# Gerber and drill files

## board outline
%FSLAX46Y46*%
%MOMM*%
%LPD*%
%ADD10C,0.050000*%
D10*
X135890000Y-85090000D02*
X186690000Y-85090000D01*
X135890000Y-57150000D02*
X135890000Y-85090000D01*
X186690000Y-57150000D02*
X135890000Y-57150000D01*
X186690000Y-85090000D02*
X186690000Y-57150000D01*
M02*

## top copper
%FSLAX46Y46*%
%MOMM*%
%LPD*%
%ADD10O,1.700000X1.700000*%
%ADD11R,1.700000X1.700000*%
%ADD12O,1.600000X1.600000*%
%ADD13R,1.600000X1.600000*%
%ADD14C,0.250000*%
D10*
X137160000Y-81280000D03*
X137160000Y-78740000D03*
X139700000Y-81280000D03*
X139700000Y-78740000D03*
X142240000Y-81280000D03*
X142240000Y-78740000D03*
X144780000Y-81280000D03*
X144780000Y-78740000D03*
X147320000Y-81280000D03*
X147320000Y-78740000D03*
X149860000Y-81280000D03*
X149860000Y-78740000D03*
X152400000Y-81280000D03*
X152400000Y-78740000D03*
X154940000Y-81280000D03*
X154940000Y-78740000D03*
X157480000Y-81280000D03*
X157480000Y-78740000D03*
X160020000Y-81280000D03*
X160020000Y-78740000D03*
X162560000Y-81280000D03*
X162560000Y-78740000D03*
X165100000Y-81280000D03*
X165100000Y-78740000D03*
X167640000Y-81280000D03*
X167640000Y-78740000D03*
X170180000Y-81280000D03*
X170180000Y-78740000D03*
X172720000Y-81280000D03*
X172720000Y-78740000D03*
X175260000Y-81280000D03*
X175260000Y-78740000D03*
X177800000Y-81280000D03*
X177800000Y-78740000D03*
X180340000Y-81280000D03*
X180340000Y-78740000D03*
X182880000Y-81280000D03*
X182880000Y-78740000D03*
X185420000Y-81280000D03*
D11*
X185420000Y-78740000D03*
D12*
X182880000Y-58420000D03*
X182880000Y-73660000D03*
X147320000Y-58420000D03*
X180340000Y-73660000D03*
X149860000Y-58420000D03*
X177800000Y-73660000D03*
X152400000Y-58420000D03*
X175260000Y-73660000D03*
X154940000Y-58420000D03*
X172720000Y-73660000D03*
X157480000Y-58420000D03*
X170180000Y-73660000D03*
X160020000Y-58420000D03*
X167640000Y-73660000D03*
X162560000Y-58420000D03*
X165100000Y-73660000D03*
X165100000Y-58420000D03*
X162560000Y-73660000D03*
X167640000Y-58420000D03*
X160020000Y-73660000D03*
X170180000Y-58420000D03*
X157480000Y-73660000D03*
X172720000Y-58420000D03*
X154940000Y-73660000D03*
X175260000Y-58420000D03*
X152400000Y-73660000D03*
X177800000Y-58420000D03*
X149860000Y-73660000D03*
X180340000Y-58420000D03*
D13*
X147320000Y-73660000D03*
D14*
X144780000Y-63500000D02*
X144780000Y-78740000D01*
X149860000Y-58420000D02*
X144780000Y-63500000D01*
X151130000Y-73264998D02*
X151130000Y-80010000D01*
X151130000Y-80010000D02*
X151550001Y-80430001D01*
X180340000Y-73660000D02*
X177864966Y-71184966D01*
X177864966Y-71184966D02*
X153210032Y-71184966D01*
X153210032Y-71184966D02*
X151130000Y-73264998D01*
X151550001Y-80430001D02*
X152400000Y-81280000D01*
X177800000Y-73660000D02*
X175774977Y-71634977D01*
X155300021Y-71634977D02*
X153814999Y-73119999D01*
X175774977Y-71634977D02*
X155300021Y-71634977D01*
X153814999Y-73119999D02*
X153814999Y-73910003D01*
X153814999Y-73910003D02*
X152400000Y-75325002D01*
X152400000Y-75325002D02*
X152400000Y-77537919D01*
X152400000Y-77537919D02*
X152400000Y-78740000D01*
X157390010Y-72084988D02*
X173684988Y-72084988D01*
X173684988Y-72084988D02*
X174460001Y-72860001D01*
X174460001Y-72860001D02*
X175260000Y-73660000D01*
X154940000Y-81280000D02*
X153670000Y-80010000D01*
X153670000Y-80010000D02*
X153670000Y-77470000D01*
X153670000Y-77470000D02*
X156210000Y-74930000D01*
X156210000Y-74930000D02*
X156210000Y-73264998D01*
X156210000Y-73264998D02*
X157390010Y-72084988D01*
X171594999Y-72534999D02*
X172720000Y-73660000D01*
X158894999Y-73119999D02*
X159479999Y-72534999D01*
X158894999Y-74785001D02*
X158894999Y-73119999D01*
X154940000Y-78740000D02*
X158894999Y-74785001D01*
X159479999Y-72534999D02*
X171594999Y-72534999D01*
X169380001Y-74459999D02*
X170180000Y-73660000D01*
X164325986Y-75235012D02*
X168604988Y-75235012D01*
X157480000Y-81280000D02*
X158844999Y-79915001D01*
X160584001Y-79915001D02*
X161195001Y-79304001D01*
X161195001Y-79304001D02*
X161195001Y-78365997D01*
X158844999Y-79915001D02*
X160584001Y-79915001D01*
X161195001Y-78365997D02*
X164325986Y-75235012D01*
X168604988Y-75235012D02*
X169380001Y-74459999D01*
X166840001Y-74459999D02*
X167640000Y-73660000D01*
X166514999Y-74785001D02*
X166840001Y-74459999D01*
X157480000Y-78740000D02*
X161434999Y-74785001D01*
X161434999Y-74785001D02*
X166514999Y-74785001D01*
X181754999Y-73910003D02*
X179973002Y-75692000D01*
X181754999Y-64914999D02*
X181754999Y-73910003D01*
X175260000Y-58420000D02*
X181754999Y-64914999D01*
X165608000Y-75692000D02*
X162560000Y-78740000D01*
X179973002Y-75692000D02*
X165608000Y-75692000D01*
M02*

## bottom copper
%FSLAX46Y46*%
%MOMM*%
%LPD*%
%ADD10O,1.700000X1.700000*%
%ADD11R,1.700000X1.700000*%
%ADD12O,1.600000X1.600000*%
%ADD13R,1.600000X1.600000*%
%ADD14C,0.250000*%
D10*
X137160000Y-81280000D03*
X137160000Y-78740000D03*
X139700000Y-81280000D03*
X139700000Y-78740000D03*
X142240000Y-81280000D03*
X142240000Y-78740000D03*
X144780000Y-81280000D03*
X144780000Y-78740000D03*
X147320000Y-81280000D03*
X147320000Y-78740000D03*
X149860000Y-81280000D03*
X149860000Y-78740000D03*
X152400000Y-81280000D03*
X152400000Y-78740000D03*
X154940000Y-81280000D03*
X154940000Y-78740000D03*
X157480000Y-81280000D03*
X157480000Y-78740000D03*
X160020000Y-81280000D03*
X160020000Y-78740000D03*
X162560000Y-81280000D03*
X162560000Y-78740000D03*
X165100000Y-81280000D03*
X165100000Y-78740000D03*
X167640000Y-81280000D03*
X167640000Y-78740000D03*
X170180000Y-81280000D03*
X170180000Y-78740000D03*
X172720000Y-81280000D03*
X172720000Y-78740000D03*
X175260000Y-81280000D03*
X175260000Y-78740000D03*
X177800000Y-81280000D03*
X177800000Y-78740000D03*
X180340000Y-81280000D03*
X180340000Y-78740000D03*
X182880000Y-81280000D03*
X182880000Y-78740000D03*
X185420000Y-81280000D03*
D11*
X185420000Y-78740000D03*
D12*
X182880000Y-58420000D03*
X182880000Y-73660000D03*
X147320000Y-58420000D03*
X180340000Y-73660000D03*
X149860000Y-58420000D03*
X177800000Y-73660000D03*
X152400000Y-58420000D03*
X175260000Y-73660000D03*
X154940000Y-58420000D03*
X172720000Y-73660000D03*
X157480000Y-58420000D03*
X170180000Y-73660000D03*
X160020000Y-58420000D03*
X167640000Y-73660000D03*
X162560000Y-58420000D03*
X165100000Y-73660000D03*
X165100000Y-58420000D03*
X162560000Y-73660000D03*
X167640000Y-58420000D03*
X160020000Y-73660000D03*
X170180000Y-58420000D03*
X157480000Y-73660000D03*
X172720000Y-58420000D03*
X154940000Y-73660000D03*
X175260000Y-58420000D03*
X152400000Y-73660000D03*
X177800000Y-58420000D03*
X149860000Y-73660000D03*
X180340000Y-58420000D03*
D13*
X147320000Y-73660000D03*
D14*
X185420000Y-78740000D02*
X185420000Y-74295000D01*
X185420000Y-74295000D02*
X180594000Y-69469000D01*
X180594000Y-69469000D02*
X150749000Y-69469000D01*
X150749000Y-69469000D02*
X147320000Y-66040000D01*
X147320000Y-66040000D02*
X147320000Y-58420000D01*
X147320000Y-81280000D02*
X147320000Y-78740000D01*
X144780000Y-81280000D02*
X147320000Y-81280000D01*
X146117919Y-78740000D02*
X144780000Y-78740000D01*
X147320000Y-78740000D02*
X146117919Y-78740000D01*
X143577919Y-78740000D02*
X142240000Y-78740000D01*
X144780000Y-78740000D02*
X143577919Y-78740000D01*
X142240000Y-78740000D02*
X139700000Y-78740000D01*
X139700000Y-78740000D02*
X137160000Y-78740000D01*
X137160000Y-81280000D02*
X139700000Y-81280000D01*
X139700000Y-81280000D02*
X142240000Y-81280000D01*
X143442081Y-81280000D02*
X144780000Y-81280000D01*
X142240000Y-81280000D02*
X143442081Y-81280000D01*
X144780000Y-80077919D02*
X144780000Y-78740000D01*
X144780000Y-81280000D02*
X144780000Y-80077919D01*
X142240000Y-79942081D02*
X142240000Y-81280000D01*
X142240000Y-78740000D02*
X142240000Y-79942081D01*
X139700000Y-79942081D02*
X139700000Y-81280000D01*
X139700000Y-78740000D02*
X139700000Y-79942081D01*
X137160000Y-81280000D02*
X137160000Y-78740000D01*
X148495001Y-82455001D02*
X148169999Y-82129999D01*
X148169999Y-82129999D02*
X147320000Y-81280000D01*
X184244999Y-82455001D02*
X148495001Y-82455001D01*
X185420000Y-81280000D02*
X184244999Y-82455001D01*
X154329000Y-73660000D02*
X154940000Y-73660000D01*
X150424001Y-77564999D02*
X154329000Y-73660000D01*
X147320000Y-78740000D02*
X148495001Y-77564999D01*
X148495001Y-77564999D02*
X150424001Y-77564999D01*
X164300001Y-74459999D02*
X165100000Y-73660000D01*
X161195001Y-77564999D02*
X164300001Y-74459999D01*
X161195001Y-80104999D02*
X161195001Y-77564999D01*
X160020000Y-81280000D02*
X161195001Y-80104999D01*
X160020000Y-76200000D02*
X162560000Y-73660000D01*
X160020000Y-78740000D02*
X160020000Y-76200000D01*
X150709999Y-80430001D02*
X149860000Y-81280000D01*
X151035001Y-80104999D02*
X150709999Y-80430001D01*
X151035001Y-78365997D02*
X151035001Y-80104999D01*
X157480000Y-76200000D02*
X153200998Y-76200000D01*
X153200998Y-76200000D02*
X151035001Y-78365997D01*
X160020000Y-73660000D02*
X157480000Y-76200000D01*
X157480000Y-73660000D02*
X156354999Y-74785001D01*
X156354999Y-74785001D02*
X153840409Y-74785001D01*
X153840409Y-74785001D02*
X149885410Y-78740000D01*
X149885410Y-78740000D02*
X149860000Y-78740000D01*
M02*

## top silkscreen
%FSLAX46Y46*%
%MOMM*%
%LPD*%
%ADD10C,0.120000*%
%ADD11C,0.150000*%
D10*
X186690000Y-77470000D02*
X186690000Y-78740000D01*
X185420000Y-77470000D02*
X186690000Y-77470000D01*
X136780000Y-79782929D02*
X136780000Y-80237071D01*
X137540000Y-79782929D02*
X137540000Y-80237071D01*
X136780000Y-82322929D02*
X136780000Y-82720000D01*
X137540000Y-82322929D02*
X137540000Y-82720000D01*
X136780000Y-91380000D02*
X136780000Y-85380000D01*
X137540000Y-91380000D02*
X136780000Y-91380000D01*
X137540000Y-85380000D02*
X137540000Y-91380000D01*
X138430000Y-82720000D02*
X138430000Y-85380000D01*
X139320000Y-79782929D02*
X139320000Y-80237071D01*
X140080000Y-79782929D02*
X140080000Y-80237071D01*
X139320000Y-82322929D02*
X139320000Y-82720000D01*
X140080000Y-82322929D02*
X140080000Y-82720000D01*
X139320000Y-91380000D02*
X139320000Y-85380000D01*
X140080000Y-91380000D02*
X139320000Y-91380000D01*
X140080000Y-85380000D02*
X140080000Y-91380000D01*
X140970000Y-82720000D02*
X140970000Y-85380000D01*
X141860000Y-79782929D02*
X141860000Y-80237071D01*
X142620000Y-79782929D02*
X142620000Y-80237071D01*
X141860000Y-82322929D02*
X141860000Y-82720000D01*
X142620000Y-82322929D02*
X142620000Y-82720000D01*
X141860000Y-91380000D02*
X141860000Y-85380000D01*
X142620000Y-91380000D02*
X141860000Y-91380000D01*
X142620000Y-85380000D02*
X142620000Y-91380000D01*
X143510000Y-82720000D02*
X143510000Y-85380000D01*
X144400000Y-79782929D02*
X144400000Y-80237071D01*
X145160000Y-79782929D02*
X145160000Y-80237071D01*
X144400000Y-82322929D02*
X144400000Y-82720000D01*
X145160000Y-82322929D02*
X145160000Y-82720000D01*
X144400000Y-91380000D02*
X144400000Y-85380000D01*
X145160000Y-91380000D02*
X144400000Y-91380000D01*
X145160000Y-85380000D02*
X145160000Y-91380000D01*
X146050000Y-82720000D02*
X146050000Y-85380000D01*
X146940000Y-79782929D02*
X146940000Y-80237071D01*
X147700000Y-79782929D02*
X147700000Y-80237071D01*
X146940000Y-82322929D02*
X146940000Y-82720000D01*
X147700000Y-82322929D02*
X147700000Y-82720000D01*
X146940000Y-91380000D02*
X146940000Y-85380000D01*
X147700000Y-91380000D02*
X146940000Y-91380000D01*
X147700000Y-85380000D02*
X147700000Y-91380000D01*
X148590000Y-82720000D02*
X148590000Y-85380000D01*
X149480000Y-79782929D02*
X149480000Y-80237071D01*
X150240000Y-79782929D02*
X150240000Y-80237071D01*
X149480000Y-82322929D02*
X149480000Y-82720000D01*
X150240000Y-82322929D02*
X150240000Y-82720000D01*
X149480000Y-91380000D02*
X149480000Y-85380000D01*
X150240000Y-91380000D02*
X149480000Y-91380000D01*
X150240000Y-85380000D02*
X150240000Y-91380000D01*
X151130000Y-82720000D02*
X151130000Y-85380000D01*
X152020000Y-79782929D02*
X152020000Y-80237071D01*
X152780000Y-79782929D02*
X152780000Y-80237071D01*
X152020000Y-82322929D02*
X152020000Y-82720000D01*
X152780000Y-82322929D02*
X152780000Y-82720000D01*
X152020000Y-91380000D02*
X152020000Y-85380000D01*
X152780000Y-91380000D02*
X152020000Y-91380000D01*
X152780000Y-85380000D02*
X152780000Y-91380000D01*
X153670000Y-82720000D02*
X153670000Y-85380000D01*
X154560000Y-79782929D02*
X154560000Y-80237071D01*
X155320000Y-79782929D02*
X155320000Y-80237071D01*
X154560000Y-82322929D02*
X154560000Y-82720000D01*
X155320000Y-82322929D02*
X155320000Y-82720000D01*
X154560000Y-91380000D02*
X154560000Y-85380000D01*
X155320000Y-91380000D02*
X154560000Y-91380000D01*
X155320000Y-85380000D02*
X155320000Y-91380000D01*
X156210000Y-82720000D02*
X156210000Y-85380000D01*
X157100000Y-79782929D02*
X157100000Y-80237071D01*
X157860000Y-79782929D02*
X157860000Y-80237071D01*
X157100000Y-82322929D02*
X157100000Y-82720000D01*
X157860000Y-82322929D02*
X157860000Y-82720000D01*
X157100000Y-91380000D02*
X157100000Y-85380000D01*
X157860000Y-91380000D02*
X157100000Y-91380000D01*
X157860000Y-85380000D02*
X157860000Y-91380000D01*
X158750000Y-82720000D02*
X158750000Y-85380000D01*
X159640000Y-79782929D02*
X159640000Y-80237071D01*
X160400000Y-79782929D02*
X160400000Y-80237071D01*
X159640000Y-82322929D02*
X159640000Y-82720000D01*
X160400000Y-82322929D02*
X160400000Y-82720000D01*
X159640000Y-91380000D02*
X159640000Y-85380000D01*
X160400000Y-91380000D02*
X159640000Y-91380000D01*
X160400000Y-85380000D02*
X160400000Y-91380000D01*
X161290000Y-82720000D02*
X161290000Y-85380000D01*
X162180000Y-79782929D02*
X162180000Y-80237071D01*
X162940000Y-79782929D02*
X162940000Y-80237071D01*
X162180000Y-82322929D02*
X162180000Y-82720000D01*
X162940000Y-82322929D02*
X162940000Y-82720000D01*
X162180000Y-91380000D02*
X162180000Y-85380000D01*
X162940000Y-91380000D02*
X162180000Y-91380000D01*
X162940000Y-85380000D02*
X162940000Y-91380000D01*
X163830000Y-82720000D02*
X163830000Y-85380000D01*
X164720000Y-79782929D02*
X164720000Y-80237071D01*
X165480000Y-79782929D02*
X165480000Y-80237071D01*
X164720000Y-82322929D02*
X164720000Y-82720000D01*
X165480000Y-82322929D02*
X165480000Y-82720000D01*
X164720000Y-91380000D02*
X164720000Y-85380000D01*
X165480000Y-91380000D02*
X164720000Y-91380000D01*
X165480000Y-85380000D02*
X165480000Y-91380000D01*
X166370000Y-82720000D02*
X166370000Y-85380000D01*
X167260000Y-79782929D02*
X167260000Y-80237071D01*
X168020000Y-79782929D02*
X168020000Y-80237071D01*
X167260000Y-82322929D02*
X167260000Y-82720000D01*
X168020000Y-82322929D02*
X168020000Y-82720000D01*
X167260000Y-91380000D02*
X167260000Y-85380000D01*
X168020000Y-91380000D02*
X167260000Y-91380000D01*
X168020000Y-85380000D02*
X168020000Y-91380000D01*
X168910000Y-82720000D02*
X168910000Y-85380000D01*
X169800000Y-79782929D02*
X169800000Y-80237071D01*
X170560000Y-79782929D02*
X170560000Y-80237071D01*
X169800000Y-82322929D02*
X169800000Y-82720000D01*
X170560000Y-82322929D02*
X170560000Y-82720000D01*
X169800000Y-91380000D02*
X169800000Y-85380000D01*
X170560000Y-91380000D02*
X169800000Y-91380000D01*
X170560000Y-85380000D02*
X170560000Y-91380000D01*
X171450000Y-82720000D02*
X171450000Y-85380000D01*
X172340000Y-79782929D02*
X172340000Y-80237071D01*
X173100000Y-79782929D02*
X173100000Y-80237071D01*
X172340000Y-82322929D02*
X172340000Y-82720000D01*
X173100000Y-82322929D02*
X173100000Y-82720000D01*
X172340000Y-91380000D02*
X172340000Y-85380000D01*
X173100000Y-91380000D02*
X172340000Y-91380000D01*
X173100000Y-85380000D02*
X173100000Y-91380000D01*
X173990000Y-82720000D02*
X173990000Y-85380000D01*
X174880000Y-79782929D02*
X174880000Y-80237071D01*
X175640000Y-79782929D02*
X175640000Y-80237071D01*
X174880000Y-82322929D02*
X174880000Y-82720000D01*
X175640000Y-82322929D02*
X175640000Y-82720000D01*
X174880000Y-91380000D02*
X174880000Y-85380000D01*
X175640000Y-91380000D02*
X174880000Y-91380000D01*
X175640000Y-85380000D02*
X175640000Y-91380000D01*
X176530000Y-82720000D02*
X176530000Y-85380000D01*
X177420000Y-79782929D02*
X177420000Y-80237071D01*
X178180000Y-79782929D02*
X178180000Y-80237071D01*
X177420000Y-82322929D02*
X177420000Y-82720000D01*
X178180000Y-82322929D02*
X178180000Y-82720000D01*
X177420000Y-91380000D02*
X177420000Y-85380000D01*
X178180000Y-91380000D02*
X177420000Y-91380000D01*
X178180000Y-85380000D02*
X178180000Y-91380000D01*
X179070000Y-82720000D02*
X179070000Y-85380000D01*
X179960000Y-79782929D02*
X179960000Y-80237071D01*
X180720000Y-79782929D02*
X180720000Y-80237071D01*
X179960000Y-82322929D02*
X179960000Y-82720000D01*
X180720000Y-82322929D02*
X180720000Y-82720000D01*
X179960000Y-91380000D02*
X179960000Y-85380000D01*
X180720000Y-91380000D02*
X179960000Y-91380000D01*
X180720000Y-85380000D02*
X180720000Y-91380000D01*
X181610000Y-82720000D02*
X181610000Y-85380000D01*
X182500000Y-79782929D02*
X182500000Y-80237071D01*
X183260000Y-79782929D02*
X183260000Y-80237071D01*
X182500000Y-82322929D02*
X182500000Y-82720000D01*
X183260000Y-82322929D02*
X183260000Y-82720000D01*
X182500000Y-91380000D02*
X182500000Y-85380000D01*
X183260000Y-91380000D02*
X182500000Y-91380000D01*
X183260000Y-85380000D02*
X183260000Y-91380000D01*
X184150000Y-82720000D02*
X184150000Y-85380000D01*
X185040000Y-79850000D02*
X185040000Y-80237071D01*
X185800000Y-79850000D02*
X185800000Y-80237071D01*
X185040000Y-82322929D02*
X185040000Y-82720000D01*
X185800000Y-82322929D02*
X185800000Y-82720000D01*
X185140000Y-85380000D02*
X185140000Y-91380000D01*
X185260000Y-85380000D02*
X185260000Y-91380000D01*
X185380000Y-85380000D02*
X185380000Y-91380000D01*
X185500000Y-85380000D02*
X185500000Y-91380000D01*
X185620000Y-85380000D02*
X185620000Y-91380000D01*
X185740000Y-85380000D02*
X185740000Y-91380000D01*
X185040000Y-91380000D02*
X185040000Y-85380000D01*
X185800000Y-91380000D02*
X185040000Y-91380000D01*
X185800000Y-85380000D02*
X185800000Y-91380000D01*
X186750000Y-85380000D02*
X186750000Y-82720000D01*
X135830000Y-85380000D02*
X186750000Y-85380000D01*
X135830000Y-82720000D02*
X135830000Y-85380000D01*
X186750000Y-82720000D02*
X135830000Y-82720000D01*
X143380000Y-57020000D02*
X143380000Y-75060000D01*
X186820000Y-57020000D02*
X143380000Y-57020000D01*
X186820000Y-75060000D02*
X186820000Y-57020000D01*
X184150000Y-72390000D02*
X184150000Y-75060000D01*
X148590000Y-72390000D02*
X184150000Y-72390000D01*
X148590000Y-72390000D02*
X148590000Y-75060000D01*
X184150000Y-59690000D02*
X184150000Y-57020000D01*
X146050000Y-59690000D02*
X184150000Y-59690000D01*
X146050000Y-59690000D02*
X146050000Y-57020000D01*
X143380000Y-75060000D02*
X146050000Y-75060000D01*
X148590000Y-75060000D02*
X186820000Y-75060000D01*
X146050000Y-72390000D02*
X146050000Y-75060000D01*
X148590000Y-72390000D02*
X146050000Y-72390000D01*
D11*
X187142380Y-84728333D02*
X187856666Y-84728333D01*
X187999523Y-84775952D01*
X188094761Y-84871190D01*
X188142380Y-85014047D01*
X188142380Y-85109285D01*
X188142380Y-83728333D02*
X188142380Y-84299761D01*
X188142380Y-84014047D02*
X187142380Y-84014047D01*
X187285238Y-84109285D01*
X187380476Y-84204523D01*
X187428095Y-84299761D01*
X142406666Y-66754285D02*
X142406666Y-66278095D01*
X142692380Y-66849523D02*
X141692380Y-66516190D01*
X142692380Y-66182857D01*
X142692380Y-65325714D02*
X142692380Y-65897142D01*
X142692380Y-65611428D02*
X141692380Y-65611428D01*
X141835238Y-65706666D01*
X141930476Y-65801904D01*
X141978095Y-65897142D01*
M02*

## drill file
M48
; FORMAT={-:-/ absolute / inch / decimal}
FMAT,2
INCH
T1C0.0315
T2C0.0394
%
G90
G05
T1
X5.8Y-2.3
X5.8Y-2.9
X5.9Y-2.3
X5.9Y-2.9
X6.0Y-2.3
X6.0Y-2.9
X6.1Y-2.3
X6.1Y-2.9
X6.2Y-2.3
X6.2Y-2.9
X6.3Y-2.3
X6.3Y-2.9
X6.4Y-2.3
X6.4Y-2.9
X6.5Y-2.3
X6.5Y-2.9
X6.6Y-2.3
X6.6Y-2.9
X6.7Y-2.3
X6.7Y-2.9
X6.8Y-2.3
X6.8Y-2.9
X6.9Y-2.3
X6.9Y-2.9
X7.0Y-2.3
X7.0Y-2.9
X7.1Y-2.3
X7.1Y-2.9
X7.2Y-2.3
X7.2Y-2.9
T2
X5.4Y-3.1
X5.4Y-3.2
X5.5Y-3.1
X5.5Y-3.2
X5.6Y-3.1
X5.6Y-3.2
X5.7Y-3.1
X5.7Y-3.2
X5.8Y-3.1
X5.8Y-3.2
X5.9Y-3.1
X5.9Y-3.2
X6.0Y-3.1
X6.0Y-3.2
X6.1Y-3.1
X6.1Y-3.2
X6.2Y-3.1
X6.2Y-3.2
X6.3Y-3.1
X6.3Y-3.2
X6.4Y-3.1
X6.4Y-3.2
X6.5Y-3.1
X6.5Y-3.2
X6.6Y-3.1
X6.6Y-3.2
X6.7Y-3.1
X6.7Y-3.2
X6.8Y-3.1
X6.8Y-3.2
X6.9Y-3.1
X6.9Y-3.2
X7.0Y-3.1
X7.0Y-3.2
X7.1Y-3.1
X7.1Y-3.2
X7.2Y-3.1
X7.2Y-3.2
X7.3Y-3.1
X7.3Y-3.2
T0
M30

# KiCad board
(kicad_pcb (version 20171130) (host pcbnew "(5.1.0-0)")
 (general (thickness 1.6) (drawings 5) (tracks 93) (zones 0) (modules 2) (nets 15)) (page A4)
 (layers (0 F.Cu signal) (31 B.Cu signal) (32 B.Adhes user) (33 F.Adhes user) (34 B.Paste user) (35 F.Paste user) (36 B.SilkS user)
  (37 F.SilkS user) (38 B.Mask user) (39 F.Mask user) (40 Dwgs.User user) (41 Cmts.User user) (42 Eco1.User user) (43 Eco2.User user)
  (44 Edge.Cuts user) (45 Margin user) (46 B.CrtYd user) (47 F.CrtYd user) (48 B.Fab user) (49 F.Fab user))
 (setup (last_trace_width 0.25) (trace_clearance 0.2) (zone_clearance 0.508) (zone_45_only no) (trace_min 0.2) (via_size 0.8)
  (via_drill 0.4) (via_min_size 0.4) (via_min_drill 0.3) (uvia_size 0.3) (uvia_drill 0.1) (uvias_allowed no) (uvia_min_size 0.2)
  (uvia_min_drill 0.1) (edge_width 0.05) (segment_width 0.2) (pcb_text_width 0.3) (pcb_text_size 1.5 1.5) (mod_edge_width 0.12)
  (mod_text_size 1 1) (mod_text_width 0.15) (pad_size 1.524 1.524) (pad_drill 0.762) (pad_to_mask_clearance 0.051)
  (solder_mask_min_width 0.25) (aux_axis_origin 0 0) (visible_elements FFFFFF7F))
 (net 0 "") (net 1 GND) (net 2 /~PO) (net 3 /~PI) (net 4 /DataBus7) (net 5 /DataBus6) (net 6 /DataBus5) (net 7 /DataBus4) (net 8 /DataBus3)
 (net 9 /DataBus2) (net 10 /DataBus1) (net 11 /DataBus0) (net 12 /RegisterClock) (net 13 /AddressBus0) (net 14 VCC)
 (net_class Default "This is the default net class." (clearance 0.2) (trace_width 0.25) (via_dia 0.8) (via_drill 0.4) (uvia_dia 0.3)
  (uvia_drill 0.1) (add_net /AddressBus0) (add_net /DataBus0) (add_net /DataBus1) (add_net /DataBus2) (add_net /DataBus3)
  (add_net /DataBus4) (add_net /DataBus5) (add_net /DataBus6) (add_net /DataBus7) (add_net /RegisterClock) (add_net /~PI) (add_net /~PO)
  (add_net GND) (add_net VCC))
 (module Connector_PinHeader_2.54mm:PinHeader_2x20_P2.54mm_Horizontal (layer F.Cu) (at 185.42 78.74 270)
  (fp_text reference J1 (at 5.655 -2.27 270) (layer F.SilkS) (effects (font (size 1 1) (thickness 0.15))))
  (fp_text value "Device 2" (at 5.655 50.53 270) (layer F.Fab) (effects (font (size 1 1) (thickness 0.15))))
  (fp_line (start -1.27 -1.27) (end 0 -1.27) (layer F.SilkS) (width 0.12))
  (fp_line (start -1.27 0) (end -1.27 -1.27) (layer F.SilkS) (width 0.12))
  (fp_line (start 1.042929 48.64) (end 1.497071 48.64) (layer F.SilkS) (width 0.12))
  (fp_line (start 1.042929 47.88) (end 1.497071 47.88) (layer F.SilkS) (width 0.12))
  (fp_line (start 3.582929 48.64) (end 3.98 48.64) (layer F.SilkS) (width 0.12))
  (fp_line (start 3.582929 47.88) (end 3.98 47.88) (layer F.SilkS) (width 0.12))
  (fp_line (start 12.64 48.64) (end 6.64 48.64) (layer F.SilkS) (width 0.12))
  (fp_line (start 12.64 47.88) (end 12.64 48.64) (layer F.SilkS) (width 0.12))
  (fp_line (start 6.64 47.88) (end 12.64 47.88) (layer F.SilkS) (width 0.12))
  (fp_line (start 3.98 46.99) (end 6.64 46.99) (layer F.SilkS) (width 0.12))
  (fp_line (start 1.042929 46.1) (end 1.497071 46.1) (layer F.SilkS) (width 0.12))
  (fp_line (start 1.042929 45.34) (end 1.497071 45.34) (layer F.SilkS) (width 0.12))
  (fp_line (start 3.582929 46.1) (end 3.98 46.1) (layer F.SilkS) (width 0.12))
  (fp_line (start 3.582929 45.34) (end 3.98 45.34) (layer F.SilkS) (width 0.12))
  (fp_line (start 12.64 46.1) (end 6.64 46.1) (layer F.SilkS) (width 0.12))
  (fp_line (start 12.64 45.34) (end 12.64 46.1) (layer F.SilkS) (width 0.12))
  (fp_line (start 6.64 45.34) (end 12.64 45.34) (layer F.SilkS) (width 0.12))
  (fp_line (start 3.98 44.45) (end 6.64 44.45) (layer F.SilkS) (width 0.12))
  (fp_line (start 1.042929 43.56) (end 1.497071 43.56) (layer F.SilkS) (width 0.12))
  (fp_line (start 1.042929 42.8) (end 1.497071 42.8) (layer F.SilkS) (width 0.12))
  (fp_line (start 3.582929 43.56) (end 3.98 43.56) (layer F.SilkS) (width 0.12))
  (fp_line (start 3.582929 42.8) (end 3.98 42.8) (layer F.SilkS) (width 0.12))
  (fp_line (start 12.64 43.56) (end 6.64 43.56) (layer F.SilkS) (width 0.12))
  (fp_line (start 12.64 42.8) (end 12.64 43.56) (layer F.SilkS) (width 0.12))
  (fp_line (start 6.64 42.8) (end 12.64 42.8) (layer F.SilkS) (width 0.12))
  (fp_line (start 3.98 41.91) (end 6.64 41.91) (layer F.SilkS) (width 0.12))
  (fp_line (start 1.042929 41.02) (end 1.497071 41.02) (layer F.SilkS) (width 0.12))
  (fp_line (start 1.042929 40.26) (end 1.497071 40.26) (layer F.SilkS) (width 0.12))
  (fp_line (start 3.582929 41.02) (end 3.98 41.02) (layer F.SilkS) (width 0.12))
  (fp_line (start 3.582929 40.26) (end 3.98 40.26) (layer F.SilkS) (width 0.12))
  (fp_line (start 12.64 41.02) (end 6.64 41.02) (layer F.SilkS) (width 0.12))
  (fp_line (start 12.64 40.26) (end 12.64 41.02) (layer F.SilkS) (width 0.12))
  (fp_line (start 6.64 40.26) (end 12.64 40.26) (layer F.SilkS) (width 0.12))
  (fp_line (start 3.98 39.37) (end 6.64 39.37) (layer F.SilkS) (width 0.12))
  (fp_line (start 1.042929 38.48) (end 1.497071 38.48) (layer F.SilkS) (width 0.12))
  (fp_line (start 1.042929 37.72) (end 1.497071 37.72) (layer F.SilkS) (width 0.12))
  (fp_line (start 3.582929 38.48) (end 3.98 38.48) (layer F.SilkS) (width 0.12))
  (fp_line (start 3.582929 37.72) (end 3.98 37.72) (layer F.SilkS) (width 0.12))
  (fp_line (start 12.64 38.48) (end 6.64 38.48) (layer F.SilkS) (width 0.12))
  (fp_line (start 12.64 37.72) (end 12.64 38.48) (layer F.SilkS) (width 0.12))
  (fp_line (start 6.64 37.72) (end 12.64 37.72) (layer F.SilkS) (width 0.12))
  (fp_line (start 3.98 36.83) (end 6.64 36.83) (layer F.SilkS) (width 0.12))
  (fp_line (start 1.042929 35.94) (end 1.497071 35.94) (layer F.SilkS) (width 0.12))
  (fp_line (start 1.042929 35.18) (end 1.497071 35.18) (layer F.SilkS) (width 0.12))
  (fp_line (start 3.582929 35.94) (end 3.98 35.94) (layer F.SilkS) (width 0.12))
  (fp_line (start 3.582929 35.18) (end 3.98 35.18) (layer F.SilkS) (width 0.12))
  (fp_line (start 12.64 35.94) (end 6.64 35.94) (layer F.SilkS) (width 0.12))
  (fp_line (start 12.64 35.18) (end 12.64 35.94) (layer F.SilkS) (width 0.12))
  (fp_line (start 6.64 35.18) (end 12.64 35.18) (layer F.SilkS) (width 0.12))
  (fp_line (start 3.98 34.29) (end 6.64 34.29) (layer F.SilkS) (width 0.12))
  (fp_line (start 1.042929 33.4) (end 1.497071 33.4) (layer F.SilkS) (width 0.12))
  (fp_line (start 1.042929 32.64) (end 1.497071 32.64) (layer F.SilkS) (width 0.12))
  (fp_line (start 3.582929 33.4) (end 3.98 33.4) (layer F.SilkS) (width 0.12))
  (fp_line (start 3.582929 32.64) (end 3.98 32.64) (layer F.SilkS) (width 0.12))
  (fp_line (start 12.64 33.4) (end 6.64 33.4) (layer F.SilkS) (width 0.12))
  (fp_line (start 12.64 32.64) (end 12.64 33.4) (layer F.SilkS) (width 0.12))
  (fp_line (start 6.64 32.64) (end 12.64 32.64) (layer F.SilkS) (width 0.12))
  (fp_line (start 3.98 31.75) (end 6.64 31.75) (layer F.SilkS) (width 0.12))
  (fp_line (start 1.042929 30.86) (end 1.497071 30.86) (layer F.SilkS) (width 0.12))
  (fp_line (start 1.042929 30.1) (end 1.497071 30.1) (layer F.SilkS) (width 0.12))
  (fp_line (start 3.582929 30.86) (end 3.98 30.86) (layer F.SilkS) (width 0.12))
  (fp_line (start 3.582929 30.1) (end 3.98 30.1) (layer F.SilkS) (width 0.12))
  (fp_line (start 12.64 30.86) (end 6.64 30.86) (layer F.SilkS) (width 0.12))
  (fp_line (start 12.64 30.1) (end 12.64 30.86) (layer F.SilkS) (width 0.12))
  (fp_line (start 6.64 30.1) (end 12.64 30.1) (layer F.SilkS) (width 0.12))
  (fp_line (start 3.98 29.21) (end 6.64 29.21) (layer F.SilkS) (width 0.12))
  (fp_line (start 1.042929 28.32) (end 1.497071 28.32) (layer F.SilkS) (width 0.12))
  (fp_line (start 1.042929 27.56) (end 1.497071 27.56) (layer F.SilkS) (width 0.12))
  (fp_line (start 3.582929 28.32) (end 3.98 28.32) (layer F.SilkS) (width 0.12))
  (fp_line (start 3.582929 27.56) (end 3.98 27.56) (layer F.SilkS) (width 0.12))
  (fp_line (start 12.64 28.32) (end 6.64 28.32) (layer F.SilkS) (width 0.12))
  (fp_line (start 12.64 27.56) (end 12.64 28.32) (layer F.SilkS) (width 0.12))
  (fp_line (start 6.64 27.56) (end 12.64 27.56) (layer F.SilkS) (width 0.12))
  (fp_line (start 3.98 26.67) (end 6.64 26.67) (layer F.SilkS) (width 0.12))
  (fp_line (start 1.042929 25.78) (end 1.497071 25.78) (layer F.SilkS) (width 0.12))
  (fp_line (start 1.042929 25.02) (end 1.497071 25.02) (layer F.SilkS) (width 0.12))
  (fp_line (start 3.582929 25.78) (end 3.98 25.78) (layer F.SilkS) (width 0.12))
  (fp_line (start 3.582929 25.02) (end 3.98 25.02) (layer F.SilkS) (width 0.12))
  (fp_line (start 12.64 25.78) (end 6.64 25.78) (layer F.SilkS) (width 0.12))
  (fp_line (start 12.64 25.02) (end 12.64 25.78) (layer F.SilkS) (width 0.12))
  (fp_line (start 6.64 25.02) (end 12.64 25.02) (layer F.SilkS) (width 0.12))
  (fp_line (start 3.98 24.13) (end 6.64 24.13) (layer F.SilkS) (width 0.12))
  (fp_line (start 1.042929 23.24) (end 1.497071 23.24) (layer F.SilkS) (width 0.12))
  (fp_line (start 1.042929 22.48) (end 1.497071 22.48) (layer F.SilkS) (width 0.12))
  (fp_line (start 3.582929 23.24) (end 3.98 23.24) (layer F.SilkS) (width 0.12))
  (fp_line (start 3.582929 22.48) (end 3.98 22.48) (layer F.SilkS) (width 0.12))
  (fp_line (start 12.64 23.24) (end 6.64 23.24) (layer F.SilkS) (width 0.12))
  (fp_line (start 12.64 22.48) (end 12.64 23.24) (layer F.SilkS) (width 0.12))
  (fp_line (start 6.64 22.48) (end 12.64 22.48) (layer F.SilkS) (width 0.12))
  (fp_line (start 3.98 21.59) (end 6.64 21.59) (layer F.SilkS) (width 0.12))
  (fp_line (start 1.042929 20.7) (end 1.497071 20.7) (layer F.SilkS) (width 0.12))
  (fp_line (start 1.042929 19.94) (end 1.497071 19.94) (layer F.SilkS) (width 0.12))
  (fp_line (start 3.582929 20.7) (end 3.98 20.7) (layer F.SilkS) (width 0.12))
  (fp_line (start 3.582929 19.94) (end 3.98 19.94) (layer F.SilkS) (width 0.12))
  (fp_line (start 12.64 20.7) (end 6.64 20.7) (layer F.SilkS) (width 0.12))
  (fp_line (start 12.64 19.94) (end 12.64 20.7) (layer F.SilkS) (width 0.12))
  (fp_line (start 6.64 19.94) (end 12.64 19.94) (layer F.SilkS) (width 0.12))
  (fp_line (start 3.98 19.05) (end 6.64 19.05) (layer F.SilkS) (width 0.12))
  (fp_line (start 1.042929 18.16) (end 1.497071 18.16) (layer F.SilkS) (width 0.12))
  (fp_line (start 1.042929 17.4) (end 1.497071 17.4) (layer F.SilkS) (width 0.12))
  (fp_line (start 3.582929 18.16) (end 3.98 18.16) (layer F.SilkS) (width 0.12))
  (fp_line (start 3.582929 17.4) (end 3.98 17.4) (layer F.SilkS) (width 0.12))
  (fp_line (start 12.64 18.16) (end 6.64 18.16) (layer F.SilkS) (width 0.12))
  (fp_line (start 12.64 17.4) (end 12.64 18.16) (layer F.SilkS) (width 0.12))
  (fp_line (start 6.64 17.4) (end 12.64 17.4) (layer F.SilkS) (width 0.12))
  (fp_line (start 3.98 16.51) (end 6.64 16.51) (layer F.SilkS) (width 0.12))
  (fp_line (start 1.042929 15.62) (end 1.497071 15.62) (layer F.SilkS) (width 0.12))
  (fp_line (start 1.042929 14.86) (end 1.497071 14.86) (layer F.SilkS) (width 0.12))
  (fp_line (start 3.582929 15.62) (end 3.98 15.62) (layer F.SilkS) (width 0.12))
  (fp_line (start 3.582929 14.86) (end 3.98 14.86) (layer F.SilkS) (width 0.12))
  (fp_line (start 12.64 15.62) (end 6.64 15.62) (layer F.SilkS) (width 0.12))
  (fp_line (start 12.64 14.86) (end 12.64 15.62) (layer F.SilkS) (width 0.12))
  (fp_line (start 6.64 14.86) (end 12.64 14.86) (layer F.SilkS) (width 0.12))
  (fp_line (start 3.98 13.97) (end 6.64 13.97) (layer F.SilkS) (width 0.12))
  (fp_line (start 1.042929 13.08) (end 1.497071 13.08) (layer F.SilkS) (width 0.12))
  (fp_line (start 1.042929 12.32) (end 1.497071 12.32) (layer F.SilkS) (width 0.12))
  (fp_line (start 3.582929 13.08) (end 3.98 13.08) (layer F.SilkS) (width 0.12))
  (fp_line (start 3.582929 12.32) (end 3.98 12.32) (layer F.SilkS) (width 0.12))
  (fp_line (start 12.64 13.08) (end 6.64 13.08) (layer F.SilkS) (width 0.12))
  (fp_line (start 12.64 12.32) (end 12.64 13.08) (layer F.SilkS) (width 0.12))
  (fp_line (start 6.64 12.32) (end 12.64 12.32) (layer F.SilkS) (width 0.12))
  (fp_line (start 3.98 11.43) (end 6.64 11.43) (layer F.SilkS) (width 0.12))
  (fp_line (start 1.042929 10.54) (end 1.497071 10.54) (layer F.SilkS) (width 0.12))
  (fp_line (start 1.042929 9.78) (end 1.497071 9.78) (layer F.SilkS) (width 0.12))
  (fp_line (start 3.582929 10.54) (end 3.98 10.54) (layer F.SilkS) (width 0.12))
  (fp_line (start 3.582929 9.78) (end 3.98 9.78) (layer F.SilkS) (width 0.12))
  (fp_line (start 12.64 10.54) (end 6.64 10.54) (layer F.SilkS) (width 0.12))
  (fp_line (start 12.64 9.78) (end 12.64 10.54) (layer F.SilkS) (width 0.12))
  (fp_line (start 6.64 9.78) (end 12.64 9.78) (layer F.SilkS) (width 0.12))
  (fp_line (start 3.98 8.89) (end 6.64 8.89) (layer F.SilkS) (width 0.12))
  (fp_line (start 1.042929 8) (end 1.497071 8) (layer F.SilkS) (width 0.12))
  (fp_line (start 1.042929 7.24) (end 1.497071 7.24) (layer F.SilkS) (width 0.12))
  (fp_line (start 3.582929 8) (end 3.98 8) (layer F.SilkS) (width 0.12))
  (fp_line (start 3.582929 7.24) (end 3.98 7.24) (layer F.SilkS) (width 0.12))
  (fp_line (start 12.64 8) (end 6.64 8) (layer F.SilkS) (width 0.12))
  (fp_line (start 12.64 7.24) (end 12.64 8) (layer F.SilkS) (width 0.12))
  (fp_line (start 6.64 7.24) (end 12.64 7.24) (layer F.SilkS) (width 0.12))
  (fp_line (start 3.98 6.35) (end 6.64 6.35) (layer F.SilkS) (width 0.12))
  (fp_line (start 1.042929 5.46) (end 1.497071 5.46) (layer F.SilkS) (width 0.12))
  (fp_line (start 1.042929 4.7) (end 1.497071 4.7) (layer F.SilkS) (width 0.12))
  (fp_line (start 3.582929 5.46) (end 3.98 5.46) (layer F.SilkS) (width 0.12))
  (fp_line (start 3.582929 4.7) (end 3.98 4.7) (layer F.SilkS) (width 0.12))
  (fp_line (start 12.64 5.46) (end 6.64 5.46) (layer F.SilkS) (width 0.12))
  (fp_line (start 12.64 4.7) (end 12.64 5.46) (layer F.SilkS) (width 0.12))
  (fp_line (start 6.64 4.7) (end 12.64 4.7) (layer F.SilkS) (width 0.12))
  (fp_line (start 3.98 3.81) (end 6.64 3.81) (layer F.SilkS) (width 0.12))
  (fp_line (start 1.042929 2.92) (end 1.497071 2.92) (layer F.SilkS) (width 0.12))
  (fp_line (start 1.042929 2.16) (end 1.497071 2.16) (layer F.SilkS) (width 0.12))
  (fp_line (start 3.582929 2.92) (end 3.98 2.92) (layer F.SilkS) (width 0.12))
  (fp_line (start 3.582929 2.16) (end 3.98 2.16) (layer F.SilkS) (width 0.12))
  (fp_line (start 12.64 2.92) (end 6.64 2.92) (layer F.SilkS) (width 0.12))
  (fp_line (start 12.64 2.16) (end 12.64 2.92) (layer F.SilkS) (width 0.12))
  (fp_line (start 6.64 2.16) (end 12.64 2.16) (layer F.SilkS) (width 0.12))
  (fp_line (start 3.98 1.27) (end 6.64 1.27) (layer F.SilkS) (width 0.12))
  (fp_line (start 1.11 0.38) (end 1.497071 0.38) (layer F.SilkS) (width 0.12))
  (fp_line (start 1.11 -0.38) (end 1.497071 -0.38) (layer F.SilkS) (width 0.12))
  (fp_line (start 3.582929 0.38) (end 3.98 0.38) (layer F.SilkS) (width 0.12))
  (fp_line (start 3.582929 -0.38) (end 3.98 -0.38) (layer F.SilkS) (width 0.12))
  (fp_line (start 6.64 0.28) (end 12.64 0.28) (layer F.SilkS) (width 0.12))
  (fp_line (start 6.64 0.16) (end 12.64 0.16) (layer F.SilkS) (width 0.12))
  (fp_line (start 6.64 0.04) (end 12.64 0.04) (layer F.SilkS) (width 0.12))
  (fp_line (start 6.64 -0.08) (end 12.64 -0.08) (layer F.SilkS) (width 0.12))
  (fp_line (start 6.64 -0.2) (end 12.64 -0.2) (layer F.SilkS) (width 0.12))
  (fp_line (start 6.64 -0.32) (end 12.64 -0.32) (layer F.SilkS) (width 0.12))
  (fp_line (start 12.64 0.38) (end 6.64 0.38) (layer F.SilkS) (width 0.12))
  (fp_line (start 12.64 -0.38) (end 12.64 0.38) (layer F.SilkS) (width 0.12))
  (fp_line (start 6.64 -0.38) (end 12.64 -0.38) (layer F.SilkS) (width 0.12))
  (fp_line (start 6.64 -1.33) (end 3.98 -1.33) (layer F.SilkS) (width 0.12))
  (fp_line (start 6.64 49.59) (end 6.64 -1.33) (layer F.SilkS) (width 0.12))
  (fp_line (start 3.98 49.59) (end 6.64 49.59) (layer F.SilkS) (width 0.12))
  (fp_line (start 3.98 -1.33) (end 3.98 49.59) (layer F.SilkS) (width 0.12))
  (pad 40 thru_hole oval (at 2.54 48.26 270) (size 1.7 1.7) (drill 1) (layers *.Cu *.Mask) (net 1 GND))
  (pad 39 thru_hole oval (at 0 48.26 270) (size 1.7 1.7) (drill 1) (layers *.Cu *.Mask) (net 1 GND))
  (pad 38 thru_hole oval (at 2.54 45.72 270) (size 1.7 1.7) (drill 1) (layers *.Cu *.Mask) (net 1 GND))
  (pad 37 thru_hole oval (at 0 45.72 270) (size 1.7 1.7) (drill 1) (layers *.Cu *.Mask) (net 1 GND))
  (pad 36 thru_hole oval (at 2.54 43.18 270) (size 1.7 1.7) (drill 1) (layers *.Cu *.Mask) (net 1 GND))
  (pad 35 thru_hole oval (at 0 43.18 270) (size 1.7 1.7) (drill 1) (layers *.Cu *.Mask) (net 1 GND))
  (pad 34 thru_hole oval (at 2.54 40.64 270) (size 1.7 1.7) (drill 1) (layers *.Cu *.Mask) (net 1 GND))
  (pad 33 thru_hole oval (at 0 40.64 270) (size 1.7 1.7) (drill 1) (layers *.Cu *.Mask) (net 1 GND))
  (pad 32 thru_hole oval (at 2.54 38.1 270) (size 1.7 1.7) (drill 1) (layers *.Cu *.Mask) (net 1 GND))
  (pad 31 thru_hole oval (at 0 38.1 270) (size 1.7 1.7) (drill 1) (layers *.Cu *.Mask) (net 1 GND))
  (pad 30 thru_hole oval (at 2.54 35.56 270) (size 1.7 1.7) (drill 1) (layers *.Cu *.Mask) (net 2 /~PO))
  (pad 29 thru_hole oval (at 0 35.56 270) (size 1.7 1.7) (drill 1) (layers *.Cu *.Mask) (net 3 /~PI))
  (pad 28 thru_hole oval (at 2.54 33.02 270) (size 1.7 1.7) (drill 1) (layers *.Cu *.Mask) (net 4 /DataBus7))
  (pad 27 thru_hole oval (at 0 33.02 270) (size 1.7 1.7) (drill 1) (layers *.Cu *.Mask) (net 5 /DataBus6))
  (pad 26 thru_hole oval (at 2.54 30.48 270) (size 1.7 1.7) (drill 1) (layers *.Cu *.Mask) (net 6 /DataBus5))
  (pad 25 thru_hole oval (at 0 30.48 270) (size 1.7 1.7) (drill 1) (layers *.Cu *.Mask) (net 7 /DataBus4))
  (pad 24 thru_hole oval (at 2.54 27.94 270) (size 1.7 1.7) (drill 1) (layers *.Cu *.Mask) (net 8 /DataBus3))
  (pad 23 thru_hole oval (at 0 27.94 270) (size 1.7 1.7) (drill 1) (layers *.Cu *.Mask) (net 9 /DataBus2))
  (pad 22 thru_hole oval (at 2.54 25.4 270) (size 1.7 1.7) (drill 1) (layers *.Cu *.Mask) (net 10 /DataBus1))
  (pad 21 thru_hole oval (at 0 25.4 270) (size 1.7 1.7) (drill 1) (layers *.Cu *.Mask) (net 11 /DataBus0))
  (pad 20 thru_hole oval (at 2.54 22.86 270) (size 1.7 1.7) (drill 1) (layers *.Cu *.Mask))
  (pad 19 thru_hole oval (at 0 22.86 270) (size 1.7 1.7) (drill 1) (layers *.Cu *.Mask) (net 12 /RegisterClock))
  (pad 18 thru_hole oval (at 2.54 20.32 270) (size 1.7 1.7) (drill 1) (layers *.Cu *.Mask))
  (pad 17 thru_hole oval (at 0 20.32 270) (size 1.7 1.7) (drill 1) (layers *.Cu *.Mask))
  (pad 16 thru_hole oval (at 2.54 17.78 270) (size 1.7 1.7) (drill 1) (layers *.Cu *.Mask))
  (pad 15 thru_hole oval (at 0 17.78 270) (size 1.7 1.7) (drill 1) (layers *.Cu *.Mask))
  (pad 14 thru_hole oval (at 2.54 15.24 270) (size 1.7 1.7) (drill 1) (layers *.Cu *.Mask))
  (pad 13 thru_hole oval (at 0 15.24 270) (size 1.7 1.7) (drill 1) (layers *.Cu *.Mask))
  (pad 12 thru_hole oval (at 2.54 12.7 270) (size 1.7 1.7) (drill 1) (layers *.Cu *.Mask))
  (pad 11 thru_hole oval (at 0 12.7 270) (size 1.7 1.7) (drill 1) (layers *.Cu *.Mask))
  (pad 10 thru_hole oval (at 2.54 10.16 270) (size 1.7 1.7) (drill 1) (layers *.Cu *.Mask))
  (pad 9 thru_hole oval (at 0 10.16 270) (size 1.7 1.7) (drill 1) (layers *.Cu *.Mask))
  (pad 8 thru_hole oval (at 2.54 7.62 270) (size 1.7 1.7) (drill 1) (layers *.Cu *.Mask))
  (pad 7 thru_hole oval (at 0 7.62 270) (size 1.7 1.7) (drill 1) (layers *.Cu *.Mask))
  (pad 6 thru_hole oval (at 2.54 5.08 270) (size 1.7 1.7) (drill 1) (layers *.Cu *.Mask))
  (pad 5 thru_hole oval (at 0 5.08 270) (size 1.7 1.7) (drill 1) (layers *.Cu *.Mask))
  (pad 4 thru_hole oval (at 2.54 2.54 270) (size 1.7 1.7) (drill 1) (layers *.Cu *.Mask))
  (pad 3 thru_hole oval (at 0 2.54 270) (size 1.7 1.7) (drill 1) (layers *.Cu *.Mask) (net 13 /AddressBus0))
  (pad 2 thru_hole oval (at 2.54 0 270) (size 1.7 1.7) (drill 1) (layers *.Cu *.Mask) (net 1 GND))
  (pad 1 thru_hole rect (at 0 0 270) (size 1.7 1.7) (drill 1) (layers *.Cu *.Mask) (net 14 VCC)))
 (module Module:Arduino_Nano (layer F.Cu) (at 147.32 73.66 90)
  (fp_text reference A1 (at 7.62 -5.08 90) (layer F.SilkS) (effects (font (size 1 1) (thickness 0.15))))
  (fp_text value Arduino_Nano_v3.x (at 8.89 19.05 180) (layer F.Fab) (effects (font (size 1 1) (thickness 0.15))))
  (fp_line (start 16.64 -3.94) (end -1.4 -3.94) (layer F.SilkS) (width 0.12))
  (fp_line (start 16.64 39.5) (end 16.64 -3.94) (layer F.SilkS) (width 0.12))
  (fp_line (start -1.4 39.5) (end 16.64 39.5) (layer F.SilkS) (width 0.12))
  (fp_line (start 1.27 36.83) (end -1.4 36.83) (layer F.SilkS) (width 0.12))
  (fp_line (start 1.27 1.27) (end 1.27 36.83) (layer F.SilkS) (width 0.12))
  (fp_line (start 1.27 1.27) (end -1.4 1.27) (layer F.SilkS) (width 0.12))
  (fp_line (start 13.97 36.83) (end 16.64 36.83) (layer F.SilkS) (width 0.12))
  (fp_line (start 13.97 -1.27) (end 13.97 36.83) (layer F.SilkS) (width 0.12))
  (fp_line (start 13.97 -1.27) (end 16.64 -1.27) (layer F.SilkS) (width 0.12))
  (fp_line (start -1.4 -3.94) (end -1.4 -1.27) (layer F.SilkS) (width 0.12))
  (fp_line (start -1.4 1.27) (end -1.4 39.5) (layer F.SilkS) (width 0.12))
  (fp_line (start 1.27 -1.27) (end -1.4 -1.27) (layer F.SilkS) (width 0.12))
  (fp_line (start 1.27 1.27) (end 1.27 -1.27) (layer F.SilkS) (width 0.12))
  (pad 16 thru_hole oval (at 15.24 35.56 90) (size 1.6 1.6) (drill 0.8) (layers *.Cu *.Mask) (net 13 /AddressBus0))
  (pad 15 thru_hole oval (at 0 35.56 90) (size 1.6 1.6) (drill 0.8) (layers *.Cu *.Mask))
  (pad 30 thru_hole oval (at 15.24 0 90) (size 1.6 1.6) (drill 0.8) (layers *.Cu *.Mask) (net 14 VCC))
  (pad 14 thru_hole oval (at 0 33.02 90) (size 1.6 1.6) (drill 0.8) (layers *.Cu *.Mask) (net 4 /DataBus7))
  (pad 29 thru_hole oval (at 15.24 2.54 90) (size 1.6 1.6) (drill 0.8) (layers *.Cu *.Mask) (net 1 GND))
  (pad 13 thru_hole oval (at 0 30.48 90) (size 1.6 1.6) (drill 0.8) (layers *.Cu *.Mask) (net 5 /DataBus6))
  (pad 28 thru_hole oval (at 15.24 5.08 90) (size 1.6 1.6) (drill 0.8) (layers *.Cu *.Mask))
  (pad 12 thru_hole oval (at 0 27.94 90) (size 1.6 1.6) (drill 0.8) (layers *.Cu *.Mask) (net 6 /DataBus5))
  (pad 27 thru_hole oval (at 15.24 7.62 90) (size 1.6 1.6) (drill 0.8) (layers *.Cu *.Mask))
  (pad 11 thru_hole oval (at 0 25.4 90) (size 1.6 1.6) (drill 0.8) (layers *.Cu *.Mask) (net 7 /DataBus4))
  (pad 26 thru_hole oval (at 15.24 10.16 90) (size 1.6 1.6) (drill 0.8) (layers *.Cu *.Mask))
  (pad 10 thru_hole oval (at 0 22.86 90) (size 1.6 1.6) (drill 0.8) (layers *.Cu *.Mask) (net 8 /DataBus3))
  (pad 25 thru_hole oval (at 15.24 12.7 90) (size 1.6 1.6) (drill 0.8) (layers *.Cu *.Mask))
  (pad 9 thru_hole oval (at 0 20.32 90) (size 1.6 1.6) (drill 0.8) (layers *.Cu *.Mask) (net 9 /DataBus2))
  (pad 24 thru_hole oval (at 15.24 15.24 90) (size 1.6 1.6) (drill 0.8) (layers *.Cu *.Mask))
  (pad 8 thru_hole oval (at 0 17.78 90) (size 1.6 1.6) (drill 0.8) (layers *.Cu *.Mask) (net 10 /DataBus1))
  (pad 23 thru_hole oval (at 15.24 17.78 90) (size 1.6 1.6) (drill 0.8) (layers *.Cu *.Mask))
  (pad 7 thru_hole oval (at 0 15.24 90) (size 1.6 1.6) (drill 0.8) (layers *.Cu *.Mask) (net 11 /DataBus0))
  (pad 22 thru_hole oval (at 15.24 20.32 90) (size 1.6 1.6) (drill 0.8) (layers *.Cu *.Mask))
  (pad 6 thru_hole oval (at 0 12.7 90) (size 1.6 1.6) (drill 0.8) (layers *.Cu *.Mask) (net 2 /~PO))
  (pad 21 thru_hole oval (at 15.24 22.86 90) (size 1.6 1.6) (drill 0.8) (layers *.Cu *.Mask))
  (pad 5 thru_hole oval (at 0 10.16 90) (size 1.6 1.6) (drill 0.8) (layers *.Cu *.Mask) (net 3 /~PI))
  (pad 20 thru_hole oval (at 15.24 25.4 90) (size 1.6 1.6) (drill 0.8) (layers *.Cu *.Mask))
  (pad 4 thru_hole oval (at 0 7.62 90) (size 1.6 1.6) (drill 0.8) (layers *.Cu *.Mask) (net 1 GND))
  (pad 19 thru_hole oval (at 15.24 27.94 90) (size 1.6 1.6) (drill 0.8) (layers *.Cu *.Mask) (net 12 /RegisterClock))
  (pad 3 thru_hole oval (at 0 5.08 90) (size 1.6 1.6) (drill 0.8) (layers *.Cu *.Mask))
  (pad 18 thru_hole oval (at 15.24 30.48 90) (size 1.6 1.6) (drill 0.8) (layers *.Cu *.Mask))
  (pad 2 thru_hole oval (at 0 2.54 90) (size 1.6 1.6) (drill 0.8) (layers *.Cu *.Mask))
  (pad 17 thru_hole oval (at 15.24 33.02 90) (size 1.6 1.6) (drill 0.8) (layers *.Cu *.Mask))
  (pad 1 thru_hole rect (at 0 0 90) (size 1.6 1.6) (drill 0.8) (layers *.Cu *.Mask)))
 (gr_line (start 135.89 85.09) (end 186.69 85.09) (layer Edge.Cuts) (width 0.05))
 (gr_line (start 135.89 57.15) (end 135.89 85.09) (layer Edge.Cuts) (width 0.05))
 (gr_line (start 186.69 57.15) (end 135.89 57.15) (layer Edge.Cuts) (width 0.05))
 (gr_line (start 186.69 85.09) (end 186.69 57.15) (layer Edge.Cuts) (width 0.05))
 (segment (start 185.42 78.74) (end 185.42 74.295) (width 0.25) (layer B.Cu) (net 14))
 (segment (start 185.42 74.295) (end 180.594 69.469) (width 0.25) (layer B.Cu) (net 14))
 (segment (start 180.594 69.469) (end 150.749 69.469) (width 0.25) (layer B.Cu) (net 14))
 (segment (start 150.749 69.469) (end 147.32 66.04) (width 0.25) (layer B.Cu) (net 14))
 (segment (start 147.32 66.04) (end 147.32 58.42) (width 0.25) (layer B.Cu) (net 14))
 (segment (start 147.32 81.28) (end 147.32 78.74) (width 0.25) (layer B.Cu) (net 1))
 (segment (start 144.78 81.28) (end 147.32 81.28) (width 0.25) (layer B.Cu) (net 1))
 (segment (start 146.117919 78.74) (end 144.78 78.74) (width 0.25) (layer B.Cu) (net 1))
 (segment (start 147.32 78.74) (end 146.117919 78.74) (width 0.25) (layer B.Cu) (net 1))
 (segment (start 143.577919 78.74) (end 142.24 78.74) (width 0.25) (layer B.Cu) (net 1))
 (segment (start 144.78 78.74) (end 143.577919 78.74) (width 0.25) (layer B.Cu) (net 1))
 (segment (start 142.24 78.74) (end 139.7 78.74) (width 0.25) (layer B.Cu) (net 1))
 (segment (start 139.7 78.74) (end 137.16 78.74) (width 0.25) (layer B.Cu) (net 1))
 (segment (start 137.16 81.28) (end 139.7 81.28) (width 0.25) (layer B.Cu) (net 1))
 (segment (start 139.7 81.28) (end 142.24 81.28) (width 0.25) (layer B.Cu) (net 1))
 (segment (start 143.442081 81.28) (end 144.78 81.28) (width 0.25) (layer B.Cu) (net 1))
 (segment (start 142.24 81.28) (end 143.442081 81.28) (width 0.25) (layer B.Cu) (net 1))
 (segment (start 144.78 80.077919) (end 144.78 78.74) (width 0.25) (layer B.Cu) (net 1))
 (segment (start 144.78 81.28) (end 144.78 80.077919) (width 0.25) (layer B.Cu) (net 1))
 (segment (start 142.24 79.942081) (end 142.24 81.28) (width 0.25) (layer B.Cu) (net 1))
 (segment (start 142.24 78.74) (end 142.24 79.942081) (width 0.25) (layer B.Cu) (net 1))
 (segment (start 139.7 79.942081) (end 139.7 81.28) (width 0.25) (layer B.Cu) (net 1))
 (segment (start 139.7 78.74) (end 139.7 79.942081) (width 0.25) (layer B.Cu) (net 1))
 (segment (start 137.16 81.28) (end 137.16 78.74) (width 0.25) (layer B.Cu) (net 1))
 (segment (start 148.495001 82.455001) (end 148.169999 82.129999) (width 0.25) (layer B.Cu) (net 1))
 (segment (start 148.169999 82.129999) (end 147.32 81.28) (width 0.25) (layer B.Cu) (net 1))
 (segment (start 184.244999 82.455001) (end 148.495001 82.455001) (width 0.25) (layer B.Cu) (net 1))
 (segment (start 185.42 81.28) (end 184.244999 82.455001) (width 0.25) (layer B.Cu) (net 1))
 (segment (start 154.329 73.66) (end 154.94 73.66) (width 0.25) (layer B.Cu) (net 1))
 (segment (start 150.424001 77.564999) (end 154.329 73.66) (width 0.25) (layer B.Cu) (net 1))
 (segment (start 147.32 78.74) (end 148.495001 77.564999) (width 0.25) (layer B.Cu) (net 1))
 (segment (start 148.495001 77.564999) (end 150.424001 77.564999) (width 0.25) (layer B.Cu) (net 1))
 (segment (start 144.78 63.5) (end 144.78 78.74) (width 0.25) (layer F.Cu) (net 1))
 (segment (start 149.86 58.42) (end 144.78 63.5) (width 0.25) (layer F.Cu) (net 1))
 (segment (start 151.13 73.264998) (end 151.13 80.01) (width 0.25) (layer F.Cu) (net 4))
 (segment (start 151.13 80.01) (end 151.550001 80.430001) (width 0.25) (layer F.Cu) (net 4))
 (segment (start 180.34 73.66) (end 177.864966 71.184966) (width 0.25) (layer F.Cu) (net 4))
 (segment (start 177.864966 71.184966) (end 153.210032 71.184966) (width 0.25) (layer F.Cu) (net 4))
 (segment (start 153.210032 71.184966) (end 151.13 73.264998) (width 0.25) (layer F.Cu) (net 4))
 (segment (start 151.550001 80.430001) (end 152.4 81.28) (width 0.25) (layer F.Cu) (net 4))
 (segment (start 177.8 73.66) (end 175.774977 71.634977) (width 0.25) (layer F.Cu) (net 5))
 (segment (start 155.300021 71.634977) (end 153.814999 73.119999) (width 0.25) (layer F.Cu) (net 5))
 (segment (start 175.774977 71.634977) (end 155.300021 71.634977) (width 0.25) (layer F.Cu) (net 5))
 (segment (start 153.814999 73.119999) (end 153.814999 73.910003) (width 0.25) (layer F.Cu) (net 5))
 (segment (start 153.814999 73.910003) (end 152.4 75.325002) (width 0.25) (layer F.Cu) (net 5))
 (segment (start 152.4 75.325002) (end 152.4 77.537919) (width 0.25) (layer F.Cu) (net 5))
 (segment (start 152.4 77.537919) (end 152.4 78.74) (width 0.25) (layer F.Cu) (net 5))
 (segment (start 157.39001 72.084988) (end 173.684988 72.084988) (width 0.25) (layer F.Cu) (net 6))
 (segment (start 173.684988 72.084988) (end 174.460001 72.860001) (width 0.25) (layer F.Cu) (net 6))
 (segment (start 174.460001 72.860001) (end 175.26 73.66) (width 0.25) (layer F.Cu) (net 6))
 (segment (start 154.94 81.28) (end 153.67 80.01) (width 0.25) (layer F.Cu) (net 6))
 (segment (start 153.67 80.01) (end 153.67 77.47) (width 0.25) (layer F.Cu) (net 6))
 (segment (start 153.67 77.47) (end 156.21 74.93) (width 0.25) (layer F.Cu) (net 6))
 (segment (start 156.21 74.93) (end 156.21 73.264998) (width 0.25) (layer F.Cu) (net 6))
 (segment (start 156.21 73.264998) (end 157.39001 72.084988) (width 0.25) (layer F.Cu) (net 6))
 (segment (start 171.594999 72.534999) (end 172.72 73.66) (width 0.25) (layer F.Cu) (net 7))
 (segment (start 158.894999 73.119999) (end 159.479999 72.534999) (width 0.25) (layer F.Cu) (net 7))
 (segment (start 158.894999 74.785001) (end 158.894999 73.119999) (width 0.25) (layer F.Cu) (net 7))
 (segment (start 154.94 78.74) (end 158.894999 74.785001) (width 0.25) (layer F.Cu) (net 7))
 (segment (start 159.479999 72.534999) (end 171.594999 72.534999) (width 0.25) (layer F.Cu) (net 7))
 (segment (start 169.380001 74.459999) (end 170.18 73.66) (width 0.25) (layer F.Cu) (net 8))
 (segment (start 164.325986 75.235012) (end 168.604988 75.235012) (width 0.25) (layer F.Cu) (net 8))
 (segment (start 157.48 81.28) (end 158.844999 79.915001) (width 0.25) (layer F.Cu) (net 8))
 (segment (start 160.584001 79.915001) (end 161.195001 79.304001) (width 0.25) (layer F.Cu) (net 8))
 (segment (start 161.195001 79.304001) (end 161.195001 78.365997) (width 0.25) (layer F.Cu) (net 8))
 (segment (start 158.844999 79.915001) (end 160.584001 79.915001) (width 0.25) (layer F.Cu) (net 8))
 (segment (start 161.195001 78.365997) (end 164.325986 75.235012) (width 0.25) (layer F.Cu) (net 8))
 (segment (start 168.604988 75.235012) (end 169.380001 74.459999) (width 0.25) (layer F.Cu) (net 8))
 (segment (start 166.840001 74.459999) (end 167.64 73.66) (width 0.25) (layer F.Cu) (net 9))
 (segment (start 166.514999 74.785001) (end 166.840001 74.459999) (width 0.25) (layer F.Cu) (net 9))
 (segment (start 157.48 78.74) (end 161.434999 74.785001) (width 0.25) (layer F.Cu) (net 9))
 (segment (start 161.434999 74.785001) (end 166.514999 74.785001) (width 0.25) (layer F.Cu) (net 9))
 (segment (start 164.300001 74.459999) (end 165.1 73.66) (width 0.25) (layer B.Cu) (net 10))
 (segment (start 161.195001 77.564999) (end 164.300001 74.459999) (width 0.25) (layer B.Cu) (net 10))
 (segment (start 161.195001 80.104999) (end 161.195001 77.564999) (width 0.25) (layer B.Cu) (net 10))
 (segment (start 160.02 81.28) (end 161.195001 80.104999) (width 0.25) (layer B.Cu) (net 10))
 (segment (start 160.02 76.2) (end 162.56 73.66) (width 0.25) (layer B.Cu) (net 11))
 (segment (start 160.02 78.74) (end 160.02 76.2) (width 0.25) (layer B.Cu) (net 11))
 (segment (start 150.709999 80.430001) (end 149.86 81.28) (width 0.25) (layer B.Cu) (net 2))
 (segment (start 151.035001 80.104999) (end 150.709999 80.430001) (width 0.25) (layer B.Cu) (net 2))
 (segment (start 151.035001 78.365997) (end 151.035001 80.104999) (width 0.25) (layer B.Cu) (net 2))
 (segment (start 157.48 76.2) (end 153.200998 76.2) (width 0.25) (layer B.Cu) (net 2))
 (segment (start 153.200998 76.2) (end 151.035001 78.365997) (width 0.25) (layer B.Cu) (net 2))
 (segment (start 160.02 73.66) (end 157.48 76.2) (width 0.25) (layer B.Cu) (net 2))
 (segment (start 157.48 73.66) (end 156.354999 74.785001) (width 0.25) (layer B.Cu) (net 3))
 (segment (start 156.354999 74.785001) (end 153.840409 74.785001) (width 0.25) (layer B.Cu) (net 3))
 (segment (start 153.840409 74.785001) (end 149.88541 78.74) (width 0.25) (layer B.Cu) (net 3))
 (segment (start 149.88541 78.74) (end 149.86 78.74) (width 0.25) (layer B.Cu) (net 3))
 (segment (start 181.754999 73.910003) (end 179.973002 75.692) (width 0.25) (layer F.Cu) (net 12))
 (segment (start 181.754999 64.914999) (end 181.754999 73.910003) (width 0.25) (layer F.Cu) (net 12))
 (segment (start 175.26 58.42) (end 181.754999 64.914999) (width 0.25) (layer F.Cu) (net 12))
 (segment (start 165.608 75.692) (end 162.56 78.74) (width 0.25) (layer F.Cu) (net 12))
 (segment (start 179.973002 75.692) (end 165.608 75.692) (width 0.25) (layer F.Cu) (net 12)))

